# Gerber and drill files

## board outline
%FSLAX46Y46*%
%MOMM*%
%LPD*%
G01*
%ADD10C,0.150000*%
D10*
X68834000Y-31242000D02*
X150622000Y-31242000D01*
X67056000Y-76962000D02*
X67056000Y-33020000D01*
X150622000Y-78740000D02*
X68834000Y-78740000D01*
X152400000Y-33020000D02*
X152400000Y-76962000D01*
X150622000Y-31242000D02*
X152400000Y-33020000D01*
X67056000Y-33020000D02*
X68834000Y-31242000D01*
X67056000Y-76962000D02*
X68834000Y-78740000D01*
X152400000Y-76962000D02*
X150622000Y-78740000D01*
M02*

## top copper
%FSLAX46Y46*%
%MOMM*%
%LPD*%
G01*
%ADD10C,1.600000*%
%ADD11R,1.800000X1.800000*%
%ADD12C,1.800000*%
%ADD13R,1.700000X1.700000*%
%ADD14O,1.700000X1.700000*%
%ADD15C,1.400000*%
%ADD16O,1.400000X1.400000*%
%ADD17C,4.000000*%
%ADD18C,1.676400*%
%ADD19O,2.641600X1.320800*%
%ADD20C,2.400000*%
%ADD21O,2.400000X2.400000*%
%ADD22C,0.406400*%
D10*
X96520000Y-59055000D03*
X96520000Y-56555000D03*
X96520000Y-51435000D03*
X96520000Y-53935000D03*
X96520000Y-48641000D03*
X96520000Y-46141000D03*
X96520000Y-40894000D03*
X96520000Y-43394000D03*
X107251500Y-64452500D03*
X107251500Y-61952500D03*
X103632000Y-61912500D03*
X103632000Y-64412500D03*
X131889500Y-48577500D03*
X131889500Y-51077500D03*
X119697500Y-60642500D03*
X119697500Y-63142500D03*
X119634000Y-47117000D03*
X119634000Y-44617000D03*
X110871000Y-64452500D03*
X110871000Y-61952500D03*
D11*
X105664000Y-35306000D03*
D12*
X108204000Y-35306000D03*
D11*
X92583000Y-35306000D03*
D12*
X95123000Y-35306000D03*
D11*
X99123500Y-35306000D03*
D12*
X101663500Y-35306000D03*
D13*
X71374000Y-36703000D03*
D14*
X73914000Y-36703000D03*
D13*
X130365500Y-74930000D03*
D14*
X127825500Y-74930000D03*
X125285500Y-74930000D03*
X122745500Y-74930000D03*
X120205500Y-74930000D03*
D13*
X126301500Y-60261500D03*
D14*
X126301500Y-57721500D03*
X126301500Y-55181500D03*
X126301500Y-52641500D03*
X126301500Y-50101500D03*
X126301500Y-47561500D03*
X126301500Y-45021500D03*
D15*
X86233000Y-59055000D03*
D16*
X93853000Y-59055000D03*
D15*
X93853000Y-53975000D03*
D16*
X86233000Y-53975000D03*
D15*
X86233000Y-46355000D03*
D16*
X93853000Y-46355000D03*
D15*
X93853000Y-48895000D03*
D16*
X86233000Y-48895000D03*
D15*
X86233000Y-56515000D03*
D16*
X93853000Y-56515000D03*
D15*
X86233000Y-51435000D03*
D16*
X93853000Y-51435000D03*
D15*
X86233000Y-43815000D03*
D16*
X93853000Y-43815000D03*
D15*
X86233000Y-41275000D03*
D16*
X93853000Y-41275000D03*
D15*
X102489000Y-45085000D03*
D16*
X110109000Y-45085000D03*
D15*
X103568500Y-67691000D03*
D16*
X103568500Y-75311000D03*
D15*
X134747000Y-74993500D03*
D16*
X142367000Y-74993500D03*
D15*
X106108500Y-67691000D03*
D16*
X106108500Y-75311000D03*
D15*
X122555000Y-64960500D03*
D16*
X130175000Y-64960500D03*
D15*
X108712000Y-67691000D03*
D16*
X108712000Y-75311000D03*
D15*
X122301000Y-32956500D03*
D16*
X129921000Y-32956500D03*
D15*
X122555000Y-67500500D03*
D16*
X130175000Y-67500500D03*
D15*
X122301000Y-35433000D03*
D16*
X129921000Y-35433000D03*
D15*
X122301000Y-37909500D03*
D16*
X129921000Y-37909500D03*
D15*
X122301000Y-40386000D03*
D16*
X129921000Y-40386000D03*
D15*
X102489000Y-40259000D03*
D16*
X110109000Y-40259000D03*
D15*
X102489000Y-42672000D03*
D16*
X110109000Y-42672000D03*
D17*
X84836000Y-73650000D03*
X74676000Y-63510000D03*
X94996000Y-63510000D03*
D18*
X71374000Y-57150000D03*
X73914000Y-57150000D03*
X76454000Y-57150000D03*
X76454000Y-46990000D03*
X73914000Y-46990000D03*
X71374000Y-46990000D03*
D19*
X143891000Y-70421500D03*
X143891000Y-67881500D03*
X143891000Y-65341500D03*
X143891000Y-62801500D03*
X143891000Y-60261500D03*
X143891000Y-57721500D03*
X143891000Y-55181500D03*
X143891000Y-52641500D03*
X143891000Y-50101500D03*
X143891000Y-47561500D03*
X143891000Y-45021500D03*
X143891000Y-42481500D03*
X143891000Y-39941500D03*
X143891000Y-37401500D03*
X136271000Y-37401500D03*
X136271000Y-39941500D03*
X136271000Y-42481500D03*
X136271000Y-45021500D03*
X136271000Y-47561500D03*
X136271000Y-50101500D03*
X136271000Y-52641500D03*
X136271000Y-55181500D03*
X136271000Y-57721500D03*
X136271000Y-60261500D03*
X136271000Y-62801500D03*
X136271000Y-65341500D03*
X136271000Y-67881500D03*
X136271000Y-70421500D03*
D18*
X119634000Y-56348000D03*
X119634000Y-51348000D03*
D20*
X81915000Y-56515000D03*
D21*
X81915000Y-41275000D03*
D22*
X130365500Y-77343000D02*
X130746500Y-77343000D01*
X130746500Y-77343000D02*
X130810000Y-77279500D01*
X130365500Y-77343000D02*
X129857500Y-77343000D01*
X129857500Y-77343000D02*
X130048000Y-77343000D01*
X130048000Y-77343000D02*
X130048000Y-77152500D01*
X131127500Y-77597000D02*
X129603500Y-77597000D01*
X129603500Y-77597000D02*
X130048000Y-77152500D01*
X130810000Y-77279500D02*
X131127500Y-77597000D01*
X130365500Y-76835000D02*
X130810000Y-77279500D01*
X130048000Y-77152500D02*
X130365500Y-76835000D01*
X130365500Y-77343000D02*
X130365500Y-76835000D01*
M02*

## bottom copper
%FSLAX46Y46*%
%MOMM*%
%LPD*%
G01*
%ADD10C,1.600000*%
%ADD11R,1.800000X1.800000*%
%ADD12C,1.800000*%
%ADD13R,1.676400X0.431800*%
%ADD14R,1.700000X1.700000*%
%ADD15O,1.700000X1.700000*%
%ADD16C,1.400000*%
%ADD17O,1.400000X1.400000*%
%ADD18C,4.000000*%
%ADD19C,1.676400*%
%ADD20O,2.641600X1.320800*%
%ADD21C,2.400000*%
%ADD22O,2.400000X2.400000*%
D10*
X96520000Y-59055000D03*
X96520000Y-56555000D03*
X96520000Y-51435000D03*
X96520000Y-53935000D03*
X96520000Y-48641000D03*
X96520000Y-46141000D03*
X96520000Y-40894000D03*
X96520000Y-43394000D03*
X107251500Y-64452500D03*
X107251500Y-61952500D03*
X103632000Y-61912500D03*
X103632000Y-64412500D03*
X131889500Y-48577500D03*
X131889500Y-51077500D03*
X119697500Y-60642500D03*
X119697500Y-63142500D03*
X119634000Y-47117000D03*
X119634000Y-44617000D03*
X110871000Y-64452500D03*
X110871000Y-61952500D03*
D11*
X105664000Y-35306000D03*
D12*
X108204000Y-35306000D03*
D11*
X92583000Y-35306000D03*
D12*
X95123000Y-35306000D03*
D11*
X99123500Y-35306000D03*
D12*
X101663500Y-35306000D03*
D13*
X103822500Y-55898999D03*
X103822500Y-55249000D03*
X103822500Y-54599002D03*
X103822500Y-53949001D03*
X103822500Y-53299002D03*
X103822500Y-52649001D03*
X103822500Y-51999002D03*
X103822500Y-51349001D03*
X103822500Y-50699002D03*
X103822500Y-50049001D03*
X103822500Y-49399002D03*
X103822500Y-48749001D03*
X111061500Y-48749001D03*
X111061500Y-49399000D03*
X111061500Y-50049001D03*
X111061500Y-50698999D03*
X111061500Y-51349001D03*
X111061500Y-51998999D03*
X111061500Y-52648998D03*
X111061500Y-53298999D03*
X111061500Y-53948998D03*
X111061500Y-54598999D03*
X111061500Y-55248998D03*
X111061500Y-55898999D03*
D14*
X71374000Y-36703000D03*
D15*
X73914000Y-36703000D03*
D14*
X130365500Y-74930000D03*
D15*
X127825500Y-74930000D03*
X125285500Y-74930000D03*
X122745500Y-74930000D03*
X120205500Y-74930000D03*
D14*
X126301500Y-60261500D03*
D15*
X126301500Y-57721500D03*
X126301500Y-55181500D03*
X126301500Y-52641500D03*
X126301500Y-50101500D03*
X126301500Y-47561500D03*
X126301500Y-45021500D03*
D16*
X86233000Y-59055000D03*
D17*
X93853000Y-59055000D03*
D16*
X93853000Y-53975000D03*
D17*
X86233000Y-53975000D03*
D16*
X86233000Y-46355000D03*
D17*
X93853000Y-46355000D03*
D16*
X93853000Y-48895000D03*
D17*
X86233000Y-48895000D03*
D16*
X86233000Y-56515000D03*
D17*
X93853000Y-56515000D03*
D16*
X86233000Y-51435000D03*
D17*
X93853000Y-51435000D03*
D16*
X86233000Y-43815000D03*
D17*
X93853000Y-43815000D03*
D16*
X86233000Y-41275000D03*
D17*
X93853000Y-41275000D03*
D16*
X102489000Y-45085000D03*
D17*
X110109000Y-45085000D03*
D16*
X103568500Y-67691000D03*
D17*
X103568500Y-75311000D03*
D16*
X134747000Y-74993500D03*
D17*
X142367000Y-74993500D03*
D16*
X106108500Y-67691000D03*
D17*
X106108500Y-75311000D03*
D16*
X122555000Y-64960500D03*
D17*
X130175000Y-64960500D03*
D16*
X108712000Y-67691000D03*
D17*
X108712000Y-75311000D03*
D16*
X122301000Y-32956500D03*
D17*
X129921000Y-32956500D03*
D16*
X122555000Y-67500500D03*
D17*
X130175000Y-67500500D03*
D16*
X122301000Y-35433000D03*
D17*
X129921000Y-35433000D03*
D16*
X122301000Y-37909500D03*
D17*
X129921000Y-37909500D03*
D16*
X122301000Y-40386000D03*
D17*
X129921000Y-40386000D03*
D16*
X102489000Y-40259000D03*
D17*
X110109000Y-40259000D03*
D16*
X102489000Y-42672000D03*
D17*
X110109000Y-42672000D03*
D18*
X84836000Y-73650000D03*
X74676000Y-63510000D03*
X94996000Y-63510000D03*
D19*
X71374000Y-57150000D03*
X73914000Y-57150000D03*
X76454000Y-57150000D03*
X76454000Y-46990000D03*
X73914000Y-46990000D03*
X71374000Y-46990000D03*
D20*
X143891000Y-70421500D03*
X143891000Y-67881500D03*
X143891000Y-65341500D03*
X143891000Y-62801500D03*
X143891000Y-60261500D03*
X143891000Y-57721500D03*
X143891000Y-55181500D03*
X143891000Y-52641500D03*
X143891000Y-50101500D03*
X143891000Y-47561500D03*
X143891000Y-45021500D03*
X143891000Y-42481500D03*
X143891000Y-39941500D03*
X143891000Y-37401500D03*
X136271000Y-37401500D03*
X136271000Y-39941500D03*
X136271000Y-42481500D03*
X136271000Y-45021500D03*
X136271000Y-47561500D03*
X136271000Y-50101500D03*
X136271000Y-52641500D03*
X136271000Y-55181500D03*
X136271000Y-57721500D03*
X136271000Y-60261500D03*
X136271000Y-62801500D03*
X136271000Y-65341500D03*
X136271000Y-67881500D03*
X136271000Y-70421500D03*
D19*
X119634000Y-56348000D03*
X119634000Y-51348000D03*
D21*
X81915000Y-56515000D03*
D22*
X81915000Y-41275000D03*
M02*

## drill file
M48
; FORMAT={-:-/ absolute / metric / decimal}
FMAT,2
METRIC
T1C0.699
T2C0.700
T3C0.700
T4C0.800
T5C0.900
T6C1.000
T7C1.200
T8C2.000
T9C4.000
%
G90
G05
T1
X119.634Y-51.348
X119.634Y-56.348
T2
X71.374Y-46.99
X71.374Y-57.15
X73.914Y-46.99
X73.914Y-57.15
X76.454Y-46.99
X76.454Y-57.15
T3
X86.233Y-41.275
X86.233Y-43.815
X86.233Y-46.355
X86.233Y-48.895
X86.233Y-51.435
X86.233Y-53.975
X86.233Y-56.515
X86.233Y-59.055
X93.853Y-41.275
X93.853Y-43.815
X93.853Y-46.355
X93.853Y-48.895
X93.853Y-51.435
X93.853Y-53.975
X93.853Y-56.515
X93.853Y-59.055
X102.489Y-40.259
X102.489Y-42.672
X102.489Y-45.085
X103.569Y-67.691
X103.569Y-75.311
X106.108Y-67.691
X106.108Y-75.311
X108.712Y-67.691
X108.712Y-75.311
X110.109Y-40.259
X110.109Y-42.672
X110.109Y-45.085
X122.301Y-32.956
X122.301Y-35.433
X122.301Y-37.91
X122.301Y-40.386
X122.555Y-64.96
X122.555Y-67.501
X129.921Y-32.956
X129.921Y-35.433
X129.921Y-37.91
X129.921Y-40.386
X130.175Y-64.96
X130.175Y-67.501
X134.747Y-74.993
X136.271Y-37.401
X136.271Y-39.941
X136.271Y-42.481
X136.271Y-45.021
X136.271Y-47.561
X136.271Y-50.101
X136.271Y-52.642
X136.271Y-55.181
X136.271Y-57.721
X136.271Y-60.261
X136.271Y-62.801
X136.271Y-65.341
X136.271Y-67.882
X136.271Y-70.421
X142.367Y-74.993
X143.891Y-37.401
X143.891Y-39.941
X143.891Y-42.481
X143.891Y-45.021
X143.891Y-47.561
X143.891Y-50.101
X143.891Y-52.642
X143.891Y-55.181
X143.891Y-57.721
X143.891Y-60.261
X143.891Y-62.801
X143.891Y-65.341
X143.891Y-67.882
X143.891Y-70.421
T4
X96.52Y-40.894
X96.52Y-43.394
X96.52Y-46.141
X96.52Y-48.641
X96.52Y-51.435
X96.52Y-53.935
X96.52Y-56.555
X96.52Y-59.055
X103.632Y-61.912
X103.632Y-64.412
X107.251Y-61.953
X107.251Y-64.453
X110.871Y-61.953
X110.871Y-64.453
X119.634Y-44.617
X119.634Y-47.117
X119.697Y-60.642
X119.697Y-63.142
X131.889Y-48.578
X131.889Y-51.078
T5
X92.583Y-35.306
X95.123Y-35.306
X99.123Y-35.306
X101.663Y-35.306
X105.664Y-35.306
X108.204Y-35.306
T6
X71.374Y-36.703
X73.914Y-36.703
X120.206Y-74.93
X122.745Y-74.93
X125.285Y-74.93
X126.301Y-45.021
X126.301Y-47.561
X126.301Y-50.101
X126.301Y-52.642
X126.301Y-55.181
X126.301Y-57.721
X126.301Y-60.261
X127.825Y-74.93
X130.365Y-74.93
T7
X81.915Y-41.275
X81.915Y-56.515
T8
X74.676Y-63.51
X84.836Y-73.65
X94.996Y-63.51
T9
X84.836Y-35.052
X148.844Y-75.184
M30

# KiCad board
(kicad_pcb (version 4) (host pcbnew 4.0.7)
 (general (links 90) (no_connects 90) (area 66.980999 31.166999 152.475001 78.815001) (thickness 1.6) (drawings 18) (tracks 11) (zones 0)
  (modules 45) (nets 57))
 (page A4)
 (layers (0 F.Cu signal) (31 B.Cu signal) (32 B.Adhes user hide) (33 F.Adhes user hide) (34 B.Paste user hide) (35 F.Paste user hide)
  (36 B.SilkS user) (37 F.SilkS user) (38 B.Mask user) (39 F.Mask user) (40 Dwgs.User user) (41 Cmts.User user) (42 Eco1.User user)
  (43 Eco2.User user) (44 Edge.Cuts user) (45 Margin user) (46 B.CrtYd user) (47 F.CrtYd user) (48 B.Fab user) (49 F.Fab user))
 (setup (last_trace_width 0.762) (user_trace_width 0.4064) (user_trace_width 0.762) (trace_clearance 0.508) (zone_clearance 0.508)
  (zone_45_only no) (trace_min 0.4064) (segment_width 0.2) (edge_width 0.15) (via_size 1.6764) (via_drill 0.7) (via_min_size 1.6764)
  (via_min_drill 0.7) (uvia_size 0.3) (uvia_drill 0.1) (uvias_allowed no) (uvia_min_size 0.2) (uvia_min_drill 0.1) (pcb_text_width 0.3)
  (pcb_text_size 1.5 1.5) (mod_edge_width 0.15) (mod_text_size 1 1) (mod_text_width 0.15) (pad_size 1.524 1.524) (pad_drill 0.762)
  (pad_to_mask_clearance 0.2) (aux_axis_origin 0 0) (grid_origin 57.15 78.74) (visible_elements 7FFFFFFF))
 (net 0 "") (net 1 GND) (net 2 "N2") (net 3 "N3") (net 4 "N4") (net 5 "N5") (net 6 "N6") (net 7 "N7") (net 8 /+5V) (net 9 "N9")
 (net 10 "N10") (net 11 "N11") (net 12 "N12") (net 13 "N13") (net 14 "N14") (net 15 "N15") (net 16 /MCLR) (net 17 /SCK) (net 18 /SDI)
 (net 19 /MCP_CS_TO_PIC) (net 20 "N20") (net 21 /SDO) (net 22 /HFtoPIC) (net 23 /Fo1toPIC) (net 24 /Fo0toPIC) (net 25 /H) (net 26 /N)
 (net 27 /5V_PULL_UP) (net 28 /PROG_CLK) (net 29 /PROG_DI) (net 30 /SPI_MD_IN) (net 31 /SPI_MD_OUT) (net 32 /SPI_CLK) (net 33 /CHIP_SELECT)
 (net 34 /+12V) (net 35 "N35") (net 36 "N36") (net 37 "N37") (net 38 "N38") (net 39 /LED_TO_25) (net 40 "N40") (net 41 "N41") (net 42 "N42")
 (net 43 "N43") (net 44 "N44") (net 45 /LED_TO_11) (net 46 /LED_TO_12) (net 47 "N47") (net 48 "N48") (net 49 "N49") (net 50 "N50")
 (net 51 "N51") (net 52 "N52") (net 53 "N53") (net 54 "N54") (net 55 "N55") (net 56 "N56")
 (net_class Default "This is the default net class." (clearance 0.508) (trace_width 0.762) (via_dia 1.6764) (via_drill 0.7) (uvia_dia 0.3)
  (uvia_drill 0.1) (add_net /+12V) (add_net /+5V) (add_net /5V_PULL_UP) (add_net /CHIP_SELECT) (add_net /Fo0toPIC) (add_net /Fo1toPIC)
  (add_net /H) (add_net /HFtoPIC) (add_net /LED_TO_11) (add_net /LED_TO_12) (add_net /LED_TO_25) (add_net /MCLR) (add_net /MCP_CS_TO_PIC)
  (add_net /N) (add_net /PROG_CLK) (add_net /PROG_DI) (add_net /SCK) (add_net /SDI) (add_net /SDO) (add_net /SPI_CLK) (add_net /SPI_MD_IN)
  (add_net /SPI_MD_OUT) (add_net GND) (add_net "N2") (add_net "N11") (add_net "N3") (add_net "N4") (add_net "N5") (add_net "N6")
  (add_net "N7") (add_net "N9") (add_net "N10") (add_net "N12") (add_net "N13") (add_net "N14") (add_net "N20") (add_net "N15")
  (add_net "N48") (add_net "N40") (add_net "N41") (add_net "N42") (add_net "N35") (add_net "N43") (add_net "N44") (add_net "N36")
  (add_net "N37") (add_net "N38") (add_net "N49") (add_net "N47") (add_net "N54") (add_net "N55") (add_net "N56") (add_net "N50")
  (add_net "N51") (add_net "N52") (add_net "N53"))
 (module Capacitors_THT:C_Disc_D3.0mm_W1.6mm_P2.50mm (layer F.Cu) (at 96.52 59.055 90)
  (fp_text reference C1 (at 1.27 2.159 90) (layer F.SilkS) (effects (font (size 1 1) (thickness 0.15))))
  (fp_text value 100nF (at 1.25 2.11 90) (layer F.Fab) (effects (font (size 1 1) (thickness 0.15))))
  (pad 1 thru_hole circle (at 0 0 90) (size 1.6 1.6) (drill 0.8) (layers *.Cu *.Mask) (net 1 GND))
  (pad 2 thru_hole circle (at 2.5 0 90) (size 1.6 1.6) (drill 0.8) (layers *.Cu *.Mask) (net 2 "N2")))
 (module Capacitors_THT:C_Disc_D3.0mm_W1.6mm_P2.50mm (layer F.Cu) (at 96.52 51.435 270)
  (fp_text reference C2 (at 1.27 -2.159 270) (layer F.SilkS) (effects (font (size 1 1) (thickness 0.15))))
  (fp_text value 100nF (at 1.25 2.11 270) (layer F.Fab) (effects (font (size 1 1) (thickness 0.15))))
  (pad 1 thru_hole circle (at 0 0 270) (size 1.6 1.6) (drill 0.8) (layers *.Cu *.Mask) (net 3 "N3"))
  (pad 2 thru_hole circle (at 2.5 0 270) (size 1.6 1.6) (drill 0.8) (layers *.Cu *.Mask) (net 1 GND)))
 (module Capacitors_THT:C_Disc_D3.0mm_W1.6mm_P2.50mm (layer F.Cu) (at 96.52 48.641 90)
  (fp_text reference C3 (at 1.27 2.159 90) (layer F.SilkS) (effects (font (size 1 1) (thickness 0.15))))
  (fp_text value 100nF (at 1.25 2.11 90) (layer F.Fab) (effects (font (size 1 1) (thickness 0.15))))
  (pad 1 thru_hole circle (at 0 0 90) (size 1.6 1.6) (drill 0.8) (layers *.Cu *.Mask) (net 1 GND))
  (pad 2 thru_hole circle (at 2.5 0 90) (size 1.6 1.6) (drill 0.8) (layers *.Cu *.Mask) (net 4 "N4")))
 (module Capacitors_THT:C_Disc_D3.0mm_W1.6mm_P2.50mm (layer F.Cu) (at 96.52 40.894 270)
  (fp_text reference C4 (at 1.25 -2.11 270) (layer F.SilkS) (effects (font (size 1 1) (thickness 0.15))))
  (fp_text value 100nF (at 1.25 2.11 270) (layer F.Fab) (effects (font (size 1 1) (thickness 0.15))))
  (pad 1 thru_hole circle (at 0 0 270) (size 1.6 1.6) (drill 0.8) (layers *.Cu *.Mask) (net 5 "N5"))
  (pad 2 thru_hole circle (at 2.5 0 270) (size 1.6 1.6) (drill 0.8) (layers *.Cu *.Mask) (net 1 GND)))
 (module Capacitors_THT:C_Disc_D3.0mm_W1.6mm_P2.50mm (layer F.Cu) (at 107.2515 64.4525 90)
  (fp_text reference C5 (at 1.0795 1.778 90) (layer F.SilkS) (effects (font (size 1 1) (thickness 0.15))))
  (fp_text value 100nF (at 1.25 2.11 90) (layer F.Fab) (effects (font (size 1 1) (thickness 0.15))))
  (pad 1 thru_hole circle (at 0 0 90) (size 1.6 1.6) (drill 0.8) (layers *.Cu *.Mask) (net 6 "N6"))
  (pad 2 thru_hole circle (at 2.5 0 90) (size 1.6 1.6) (drill 0.8) (layers *.Cu *.Mask) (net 1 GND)))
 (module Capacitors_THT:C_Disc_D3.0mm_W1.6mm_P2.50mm (layer F.Cu) (at 103.632 61.9125 270)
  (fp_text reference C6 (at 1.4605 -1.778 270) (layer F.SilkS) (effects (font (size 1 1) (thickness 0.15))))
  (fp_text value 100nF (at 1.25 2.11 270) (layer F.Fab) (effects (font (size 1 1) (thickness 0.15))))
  (pad 1 thru_hole circle (at 0 0 270) (size 1.6 1.6) (drill 0.8) (layers *.Cu *.Mask) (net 1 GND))
  (pad 2 thru_hole circle (at 2.5 0 270) (size 1.6 1.6) (drill 0.8) (layers *.Cu *.Mask) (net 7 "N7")))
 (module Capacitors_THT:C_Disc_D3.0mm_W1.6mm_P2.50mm (layer F.Cu) (at 131.8895 48.5775 270)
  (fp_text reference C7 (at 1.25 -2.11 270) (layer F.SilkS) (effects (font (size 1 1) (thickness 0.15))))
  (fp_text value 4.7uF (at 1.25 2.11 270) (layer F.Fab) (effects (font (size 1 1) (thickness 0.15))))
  (pad 1 thru_hole circle (at 0 0 270) (size 1.6 1.6) (drill 0.8) (layers *.Cu *.Mask) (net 1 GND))
  (pad 2 thru_hole circle (at 2.5 0 270) (size 1.6 1.6) (drill 0.8) (layers *.Cu *.Mask) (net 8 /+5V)))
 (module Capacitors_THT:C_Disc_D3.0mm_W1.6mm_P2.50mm (layer F.Cu) (at 119.6975 60.6425 270)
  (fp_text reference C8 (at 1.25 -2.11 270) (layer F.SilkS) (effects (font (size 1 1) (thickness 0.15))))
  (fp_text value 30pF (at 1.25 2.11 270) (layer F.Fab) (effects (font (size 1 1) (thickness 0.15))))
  (pad 1 thru_hole circle (at 0 0 270) (size 1.6 1.6) (drill 0.8) (layers *.Cu *.Mask) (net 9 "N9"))
  (pad 2 thru_hole circle (at 2.5 0 270) (size 1.6 1.6) (drill 0.8) (layers *.Cu *.Mask) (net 1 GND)))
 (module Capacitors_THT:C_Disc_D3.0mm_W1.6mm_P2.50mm (layer F.Cu) (at 119.634 47.117 90)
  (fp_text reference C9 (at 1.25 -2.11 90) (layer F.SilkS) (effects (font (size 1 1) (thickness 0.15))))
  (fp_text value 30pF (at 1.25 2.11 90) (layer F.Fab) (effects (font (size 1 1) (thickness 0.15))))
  (pad 1 thru_hole circle (at 0 0 90) (size 1.6 1.6) (drill 0.8) (layers *.Cu *.Mask) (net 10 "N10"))
  (pad 2 thru_hole circle (at 2.5 0 90) (size 1.6 1.6) (drill 0.8) (layers *.Cu *.Mask) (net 1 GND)))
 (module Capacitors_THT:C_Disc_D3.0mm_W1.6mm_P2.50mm (layer F.Cu) (at 110.871 64.4525 90)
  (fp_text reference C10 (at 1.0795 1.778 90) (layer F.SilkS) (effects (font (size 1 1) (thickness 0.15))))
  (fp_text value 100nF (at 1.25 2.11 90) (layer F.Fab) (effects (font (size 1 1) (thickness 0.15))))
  (pad 1 thru_hole circle (at 0 0 90) (size 1.6 1.6) (drill 0.8) (layers *.Cu *.Mask) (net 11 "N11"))
  (pad 2 thru_hole circle (at 2.5 0 90) (size 1.6 1.6) (drill 0.8) (layers *.Cu *.Mask) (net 1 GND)))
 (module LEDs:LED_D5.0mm (layer F.Cu) (at 105.664 35.306)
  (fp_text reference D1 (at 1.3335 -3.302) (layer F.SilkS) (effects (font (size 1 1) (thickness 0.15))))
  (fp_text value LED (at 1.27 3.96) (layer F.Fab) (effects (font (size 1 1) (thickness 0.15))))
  (pad 1 thru_hole rect (at 0 0) (size 1.8 1.8) (drill 0.9) (layers *.Cu *.Mask) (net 1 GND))
  (pad 2 thru_hole circle (at 2.54 0) (size 1.8 1.8) (drill 0.9) (layers *.Cu *.Mask) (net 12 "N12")))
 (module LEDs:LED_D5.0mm (layer F.Cu) (at 92.583 35.306)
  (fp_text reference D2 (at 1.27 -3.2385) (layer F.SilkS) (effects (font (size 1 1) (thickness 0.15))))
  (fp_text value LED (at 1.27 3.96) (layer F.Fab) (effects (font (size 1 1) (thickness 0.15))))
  (pad 1 thru_hole rect (at 0 0) (size 1.8 1.8) (drill 0.9) (layers *.Cu *.Mask) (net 1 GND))
  (pad 2 thru_hole circle (at 2.54 0) (size 1.8 1.8) (drill 0.9) (layers *.Cu *.Mask) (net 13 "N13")))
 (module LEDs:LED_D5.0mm (layer F.Cu) (at 99.1235 35.306)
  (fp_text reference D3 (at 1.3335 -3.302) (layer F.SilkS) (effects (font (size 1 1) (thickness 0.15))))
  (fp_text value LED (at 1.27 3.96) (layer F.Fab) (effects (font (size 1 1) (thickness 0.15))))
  (pad 1 thru_hole rect (at 0 0) (size 1.8 1.8) (drill 0.9) (layers *.Cu *.Mask) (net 1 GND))
  (pad 2 thru_hole circle (at 2.54 0) (size 1.8 1.8) (drill 0.9) (layers *.Cu *.Mask) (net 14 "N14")))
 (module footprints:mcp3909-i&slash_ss (layer B.Cu) (at 107.442 52.324)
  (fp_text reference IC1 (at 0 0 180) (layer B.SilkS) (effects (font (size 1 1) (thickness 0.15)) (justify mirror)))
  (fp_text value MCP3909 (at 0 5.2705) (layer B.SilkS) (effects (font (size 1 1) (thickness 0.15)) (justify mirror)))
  (pad 1 smd rect (at -3.6195 3.574999) (size 1.6764 0.4318) (layers B.Cu B.Paste B.Mask) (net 7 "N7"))
  (pad 2 smd rect (at -3.6195 2.925) (size 1.6764 0.4318) (layers B.Cu B.Paste B.Mask) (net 7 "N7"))
  (pad 3 smd rect (at -3.6195 2.275002) (size 1.6764 0.4318) (layers B.Cu B.Paste B.Mask) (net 7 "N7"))
  (pad 4 smd rect (at -3.6195 1.625001) (size 1.6764 0.4318) (layers B.Cu B.Paste B.Mask) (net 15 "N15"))
  (pad 5 smd rect (at -3.6195 0.975002) (size 1.6764 0.4318) (layers B.Cu B.Paste B.Mask) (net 2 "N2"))
  (pad 6 smd rect (at -3.6195 0.325001) (size 1.6764 0.4318) (layers B.Cu B.Paste B.Mask) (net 3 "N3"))
  (pad 7 smd rect (at -3.6195 -0.324998) (size 1.6764 0.4318) (layers B.Cu B.Paste B.Mask) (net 4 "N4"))
  (pad 8 smd rect (at -3.6195 -0.974999) (size 1.6764 0.4318) (layers B.Cu B.Paste B.Mask) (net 5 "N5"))
  (pad 9 smd rect (at -3.6195 -1.624998) (size 1.6764 0.4318) (layers B.Cu B.Paste B.Mask) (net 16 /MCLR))
  (pad 10 smd rect (at -3.6195 -2.274999) (size 1.6764 0.4318) (layers B.Cu B.Paste B.Mask) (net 6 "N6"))
  (pad 11 smd rect (at -3.6195 -2.924998) (size 1.6764 0.4318) (layers B.Cu B.Paste B.Mask) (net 1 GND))
  (pad 12 smd rect (at -3.6195 -3.574999) (size 1.6764 0.4318) (layers B.Cu B.Paste B.Mask) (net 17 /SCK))
  (pad 13 smd rect (at 3.6195 -3.574999) (size 1.6764 0.4318) (layers B.Cu B.Paste B.Mask) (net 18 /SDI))
  (pad 14 smd rect (at 3.6195 -2.925) (size 1.6764 0.4318) (layers B.Cu B.Paste B.Mask) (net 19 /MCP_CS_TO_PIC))
  (pad 15 smd rect (at 3.6195 -2.274999) (size 1.6764 0.4318) (layers B.Cu B.Paste B.Mask) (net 1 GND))
  (pad 16 smd rect (at 3.6195 -1.625001) (size 1.6764 0.4318) (layers B.Cu B.Paste B.Mask) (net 1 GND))
  (pad 17 smd rect (at 3.6195 -0.974999) (size 1.6764 0.4318) (layers B.Cu B.Paste B.Mask) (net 10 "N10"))
  (pad 18 smd rect (at 3.6195 -0.325001) (size 1.6764 0.4318) (layers B.Cu B.Paste B.Mask) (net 9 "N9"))
  (pad 19 smd rect (at 3.6195 0.324998) (size 1.6764 0.4318) (layers B.Cu B.Paste B.Mask) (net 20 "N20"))
  (pad 20 smd rect (at 3.6195 0.974999) (size 1.6764 0.4318) (layers B.Cu B.Paste B.Mask) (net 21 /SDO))
  (pad 21 smd rect (at 3.6195 1.624998) (size 1.6764 0.4318) (layers B.Cu B.Paste B.Mask) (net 1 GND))
  (pad 22 smd rect (at 3.6195 2.274999) (size 1.6764 0.4318) (layers B.Cu B.Paste B.Mask) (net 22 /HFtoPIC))
  (pad 23 smd rect (at 3.6195 2.924998) (size 1.6764 0.4318) (layers B.Cu B.Paste B.Mask) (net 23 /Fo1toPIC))
  (pad 24 smd rect (at 3.6195 3.574999) (size 1.6764 0.4318) (layers B.Cu B.Paste B.Mask) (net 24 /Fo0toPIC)))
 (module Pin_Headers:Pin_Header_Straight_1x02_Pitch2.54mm (layer F.Cu) (at 71.374 36.703 90)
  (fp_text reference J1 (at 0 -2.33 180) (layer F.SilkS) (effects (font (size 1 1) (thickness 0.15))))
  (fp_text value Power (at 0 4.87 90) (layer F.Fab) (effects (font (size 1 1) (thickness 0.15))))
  (pad 1 thru_hole rect (at 0 0 90) (size 1.7 1.7) (drill 1) (layers *.Cu *.Mask) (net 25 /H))
  (pad 2 thru_hole oval (at 0 2.54 90) (size 1.7 1.7) (drill 1) (layers *.Cu *.Mask) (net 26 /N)))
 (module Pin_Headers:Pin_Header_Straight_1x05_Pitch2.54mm (layer F.Cu) (at 130.3655 74.93 270)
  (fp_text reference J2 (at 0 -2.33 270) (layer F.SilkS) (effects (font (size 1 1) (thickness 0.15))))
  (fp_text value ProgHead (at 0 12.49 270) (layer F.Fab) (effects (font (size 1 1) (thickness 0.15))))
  (pad 1 thru_hole rect (at 0 0 270) (size 1.7 1.7) (drill 1) (layers *.Cu *.Mask) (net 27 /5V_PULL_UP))
  (pad 2 thru_hole oval (at 0 2.54 270) (size 1.7 1.7) (drill 1) (layers *.Cu *.Mask) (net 8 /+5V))
  (pad 3 thru_hole oval (at 0 5.08 270) (size 1.7 1.7) (drill 1) (layers *.Cu *.Mask) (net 1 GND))
  (pad 4 thru_hole oval (at 0 7.62 270) (size 1.7 1.7) (drill 1) (layers *.Cu *.Mask) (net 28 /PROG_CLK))
  (pad 5 thru_hole oval (at 0 10.16 270) (size 1.7 1.7) (drill 1) (layers *.Cu *.Mask) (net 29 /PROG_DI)))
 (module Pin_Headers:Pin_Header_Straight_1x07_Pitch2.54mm (layer F.Cu) (at 126.3015 60.2615 180)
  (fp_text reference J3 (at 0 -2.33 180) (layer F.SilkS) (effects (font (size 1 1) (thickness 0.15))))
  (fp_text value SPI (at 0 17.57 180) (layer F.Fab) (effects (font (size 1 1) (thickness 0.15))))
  (pad 1 thru_hole rect (at 0 0 180) (size 1.7 1.7) (drill 1) (layers *.Cu *.Mask) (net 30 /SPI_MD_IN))
  (pad 2 thru_hole oval (at 0 2.54 180) (size 1.7 1.7) (drill 1) (layers *.Cu *.Mask) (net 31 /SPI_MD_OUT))
  (pad 3 thru_hole oval (at 0 5.08 180) (size 1.7 1.7) (drill 1) (layers *.Cu *.Mask) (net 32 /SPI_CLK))
  (pad 4 thru_hole oval (at 0 7.62 180) (size 1.7 1.7) (drill 1) (layers *.Cu *.Mask) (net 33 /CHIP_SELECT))
  (pad 5 thru_hole oval (at 0 10.16 180) (size 1.7 1.7) (drill 1) (layers *.Cu *.Mask) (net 8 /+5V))
  (pad 6 thru_hole oval (at 0 12.7 180) (size 1.7 1.7) (drill 1) (layers *.Cu *.Mask) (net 1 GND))
  (pad 7 thru_hole oval (at 0 15.24 180) (size 1.7 1.7) (drill 1) (layers *.Cu *.Mask) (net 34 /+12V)))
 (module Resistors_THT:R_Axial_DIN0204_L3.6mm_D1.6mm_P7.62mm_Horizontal (layer F.Cu) (at 86.233 59.055)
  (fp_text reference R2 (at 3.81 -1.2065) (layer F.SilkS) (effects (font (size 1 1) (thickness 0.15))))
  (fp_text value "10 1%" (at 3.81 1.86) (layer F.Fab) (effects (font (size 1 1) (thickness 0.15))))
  (pad 1 thru_hole circle (at 0 0) (size 1.4 1.4) (drill 0.7) (layers *.Cu *.Mask) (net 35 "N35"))
  (pad 2 thru_hole oval (at 7.62 0) (size 1.4 1.4) (drill 0.7) (layers *.Cu *.Mask) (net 1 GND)))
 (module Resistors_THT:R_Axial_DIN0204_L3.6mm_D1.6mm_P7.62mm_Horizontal (layer F.Cu) (at 93.853 53.975 180)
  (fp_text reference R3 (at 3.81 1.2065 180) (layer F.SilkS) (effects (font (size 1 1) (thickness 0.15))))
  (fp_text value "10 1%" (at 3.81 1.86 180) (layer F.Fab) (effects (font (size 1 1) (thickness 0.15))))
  (pad 1 thru_hole circle (at 0 0 180) (size 1.4 1.4) (drill 0.7) (layers *.Cu *.Mask) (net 1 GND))
  (pad 2 thru_hole oval (at 7.62 0 180) (size 1.4 1.4) (drill 0.7) (layers *.Cu *.Mask) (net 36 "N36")))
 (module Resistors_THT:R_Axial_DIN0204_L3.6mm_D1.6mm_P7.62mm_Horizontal (layer F.Cu) (at 86.233 46.355)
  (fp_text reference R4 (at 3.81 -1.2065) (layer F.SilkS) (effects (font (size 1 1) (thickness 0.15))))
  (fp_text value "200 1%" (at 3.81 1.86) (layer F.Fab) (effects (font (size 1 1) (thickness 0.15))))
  (pad 1 thru_hole circle (at 0 0) (size 1.4 1.4) (drill 0.7) (layers *.Cu *.Mask) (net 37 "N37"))
  (pad 2 thru_hole oval (at 7.62 0) (size 1.4 1.4) (drill 0.7) (layers *.Cu *.Mask) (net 1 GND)))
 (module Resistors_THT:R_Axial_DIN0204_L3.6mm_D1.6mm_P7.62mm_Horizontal (layer F.Cu) (at 93.853 48.895 180)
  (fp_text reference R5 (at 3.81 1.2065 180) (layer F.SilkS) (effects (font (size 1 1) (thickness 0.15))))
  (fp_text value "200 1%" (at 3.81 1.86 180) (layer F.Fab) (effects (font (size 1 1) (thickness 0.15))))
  (pad 1 thru_hole circle (at 0 0 180) (size 1.4 1.4) (drill 0.7) (layers *.Cu *.Mask) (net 1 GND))
  (pad 2 thru_hole oval (at 7.62 0 180) (size 1.4 1.4) (drill 0.7) (layers *.Cu *.Mask) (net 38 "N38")))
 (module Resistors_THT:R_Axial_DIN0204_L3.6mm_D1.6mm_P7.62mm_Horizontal (layer F.Cu) (at 86.233 56.515)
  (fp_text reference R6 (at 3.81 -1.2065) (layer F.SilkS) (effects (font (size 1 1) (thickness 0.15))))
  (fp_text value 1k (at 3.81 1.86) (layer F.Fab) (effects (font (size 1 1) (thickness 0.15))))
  (pad 1 thru_hole circle (at 0 0) (size 1.4 1.4) (drill 0.7) (layers *.Cu *.Mask) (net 35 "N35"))
  (pad 2 thru_hole oval (at 7.62 0) (size 1.4 1.4) (drill 0.7) (layers *.Cu *.Mask) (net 2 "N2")))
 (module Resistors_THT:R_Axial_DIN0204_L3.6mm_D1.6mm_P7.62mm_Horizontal (layer F.Cu) (at 86.233 51.435)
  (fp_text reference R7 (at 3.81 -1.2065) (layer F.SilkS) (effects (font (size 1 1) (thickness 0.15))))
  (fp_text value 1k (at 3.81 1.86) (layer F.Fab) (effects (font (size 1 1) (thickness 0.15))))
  (pad 1 thru_hole circle (at 0 0) (size 1.4 1.4) (drill 0.7) (layers *.Cu *.Mask) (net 36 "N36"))
  (pad 2 thru_hole oval (at 7.62 0) (size 1.4 1.4) (drill 0.7) (layers *.Cu *.Mask) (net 3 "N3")))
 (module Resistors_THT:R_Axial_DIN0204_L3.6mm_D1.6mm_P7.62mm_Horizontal (layer F.Cu) (at 86.233 43.815)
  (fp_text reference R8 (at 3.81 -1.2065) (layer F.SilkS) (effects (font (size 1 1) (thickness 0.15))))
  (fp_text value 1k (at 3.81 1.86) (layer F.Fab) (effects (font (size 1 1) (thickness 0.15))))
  (pad 1 thru_hole circle (at 0 0) (size 1.4 1.4) (drill 0.7) (layers *.Cu *.Mask) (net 37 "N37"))
  (pad 2 thru_hole oval (at 7.62 0) (size 1.4 1.4) (drill 0.7) (layers *.Cu *.Mask) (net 4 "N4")))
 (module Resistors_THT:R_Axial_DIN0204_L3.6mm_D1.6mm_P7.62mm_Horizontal (layer F.Cu) (at 86.233 41.275)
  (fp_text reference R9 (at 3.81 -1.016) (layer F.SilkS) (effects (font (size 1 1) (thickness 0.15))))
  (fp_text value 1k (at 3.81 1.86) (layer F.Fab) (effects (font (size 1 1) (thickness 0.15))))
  (pad 1 thru_hole circle (at 0 0) (size 1.4 1.4) (drill 0.7) (layers *.Cu *.Mask) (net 38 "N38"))
  (pad 2 thru_hole oval (at 7.62 0) (size 1.4 1.4) (drill 0.7) (layers *.Cu *.Mask) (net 5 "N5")))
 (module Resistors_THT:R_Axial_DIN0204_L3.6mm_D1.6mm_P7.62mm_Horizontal (layer F.Cu) (at 102.489 45.085)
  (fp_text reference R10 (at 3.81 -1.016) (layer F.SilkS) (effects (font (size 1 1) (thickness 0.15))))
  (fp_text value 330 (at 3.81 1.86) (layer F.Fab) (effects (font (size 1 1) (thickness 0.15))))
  (pad 1 thru_hole circle (at 0 0) (size 1.4 1.4) (drill 0.7) (layers *.Cu *.Mask) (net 12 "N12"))
  (pad 2 thru_hole oval (at 7.62 0) (size 1.4 1.4) (drill 0.7) (layers *.Cu *.Mask) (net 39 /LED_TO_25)))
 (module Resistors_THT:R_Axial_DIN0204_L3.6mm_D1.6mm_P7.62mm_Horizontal (layer F.Cu) (at 103.5685 67.691 270)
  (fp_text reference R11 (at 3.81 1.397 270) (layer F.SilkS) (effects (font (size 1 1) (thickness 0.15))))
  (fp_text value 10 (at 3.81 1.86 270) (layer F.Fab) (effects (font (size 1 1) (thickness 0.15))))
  (pad 1 thru_hole circle (at 0 0 270) (size 1.4 1.4) (drill 0.7) (layers *.Cu *.Mask) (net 7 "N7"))
  (pad 2 thru_hole oval (at 7.62 0 270) (size 1.4 1.4) (drill 0.7) (layers *.Cu *.Mask) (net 8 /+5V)))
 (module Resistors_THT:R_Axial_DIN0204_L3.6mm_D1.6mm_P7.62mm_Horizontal (layer F.Cu) (at 134.747 74.9935)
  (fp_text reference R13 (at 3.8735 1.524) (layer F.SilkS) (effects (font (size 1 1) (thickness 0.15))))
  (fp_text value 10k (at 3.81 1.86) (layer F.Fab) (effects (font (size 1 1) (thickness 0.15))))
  (pad 1 thru_hole circle (at 0 0) (size 1.4 1.4) (drill 0.7) (layers *.Cu *.Mask) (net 8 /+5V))
  (pad 2 thru_hole oval (at 7.62 0) (size 1.4 1.4) (drill 0.7) (layers *.Cu *.Mask) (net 27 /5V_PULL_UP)))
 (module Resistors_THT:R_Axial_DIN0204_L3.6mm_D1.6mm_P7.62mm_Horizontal (layer F.Cu) (at 106.1085 67.691 270)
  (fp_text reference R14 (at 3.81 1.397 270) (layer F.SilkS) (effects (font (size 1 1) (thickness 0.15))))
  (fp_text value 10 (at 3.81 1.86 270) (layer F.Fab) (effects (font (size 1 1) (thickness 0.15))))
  (pad 1 thru_hole circle (at 0 0 270) (size 1.4 1.4) (drill 0.7) (layers *.Cu *.Mask) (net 11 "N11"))
  (pad 2 thru_hole oval (at 7.62 0 270) (size 1.4 1.4) (drill 0.7) (layers *.Cu *.Mask) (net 8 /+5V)))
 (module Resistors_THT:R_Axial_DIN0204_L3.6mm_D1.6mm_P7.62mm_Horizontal (layer F.Cu) (at 122.555 64.9605)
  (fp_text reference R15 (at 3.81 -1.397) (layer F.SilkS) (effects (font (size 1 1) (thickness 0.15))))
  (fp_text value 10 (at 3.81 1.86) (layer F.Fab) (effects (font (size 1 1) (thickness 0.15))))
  (pad 1 thru_hole circle (at 0 0) (size 1.4 1.4) (drill 0.7) (layers *.Cu *.Mask) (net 30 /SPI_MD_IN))
  (pad 2 thru_hole oval (at 7.62 0) (size 1.4 1.4) (drill 0.7) (layers *.Cu *.Mask) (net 8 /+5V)))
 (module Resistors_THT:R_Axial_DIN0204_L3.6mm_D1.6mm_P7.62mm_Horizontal (layer F.Cu) (at 108.712 67.691 270)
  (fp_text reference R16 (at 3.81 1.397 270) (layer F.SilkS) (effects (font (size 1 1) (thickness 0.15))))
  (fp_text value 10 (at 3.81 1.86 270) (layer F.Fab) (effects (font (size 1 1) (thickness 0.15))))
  (pad 1 thru_hole circle (at 0 0 270) (size 1.4 1.4) (drill 0.7) (layers *.Cu *.Mask) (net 32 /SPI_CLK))
  (pad 2 thru_hole oval (at 7.62 0 270) (size 1.4 1.4) (drill 0.7) (layers *.Cu *.Mask) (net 8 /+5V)))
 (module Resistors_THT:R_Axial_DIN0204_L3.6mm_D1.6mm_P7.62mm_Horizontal (layer F.Cu) (at 122.301 32.9565)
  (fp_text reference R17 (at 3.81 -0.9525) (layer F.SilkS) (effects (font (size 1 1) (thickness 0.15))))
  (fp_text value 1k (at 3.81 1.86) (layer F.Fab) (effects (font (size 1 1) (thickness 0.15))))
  (pad 1 thru_hole circle (at 0 0) (size 1.4 1.4) (drill 0.7) (layers *.Cu *.Mask) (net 17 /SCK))
  (pad 2 thru_hole oval (at 7.62 0) (size 1.4 1.4) (drill 0.7) (layers *.Cu *.Mask) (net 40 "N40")))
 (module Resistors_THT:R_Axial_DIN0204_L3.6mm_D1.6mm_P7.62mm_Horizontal (layer F.Cu) (at 122.555 67.5005)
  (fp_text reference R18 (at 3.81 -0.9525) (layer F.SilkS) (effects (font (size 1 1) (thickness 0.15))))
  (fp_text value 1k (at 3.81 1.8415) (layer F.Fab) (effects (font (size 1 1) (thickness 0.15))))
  (pad 1 thru_hole circle (at 0 0) (size 1.4 1.4) (drill 0.7) (layers *.Cu *.Mask) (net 18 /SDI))
  (pad 2 thru_hole oval (at 7.62 0) (size 1.4 1.4) (drill 0.7) (layers *.Cu *.Mask) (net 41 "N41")))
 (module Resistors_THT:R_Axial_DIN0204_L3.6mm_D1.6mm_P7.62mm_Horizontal (layer F.Cu) (at 122.301 35.433)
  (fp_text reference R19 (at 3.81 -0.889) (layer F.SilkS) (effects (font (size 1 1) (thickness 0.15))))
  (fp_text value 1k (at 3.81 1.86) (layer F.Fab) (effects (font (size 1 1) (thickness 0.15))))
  (pad 1 thru_hole circle (at 0 0) (size 1.4 1.4) (drill 0.7) (layers *.Cu *.Mask) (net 21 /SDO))
  (pad 2 thru_hole oval (at 7.62 0) (size 1.4 1.4) (drill 0.7) (layers *.Cu *.Mask) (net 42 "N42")))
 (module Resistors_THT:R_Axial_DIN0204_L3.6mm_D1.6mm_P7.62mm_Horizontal (layer F.Cu) (at 122.301 37.9095)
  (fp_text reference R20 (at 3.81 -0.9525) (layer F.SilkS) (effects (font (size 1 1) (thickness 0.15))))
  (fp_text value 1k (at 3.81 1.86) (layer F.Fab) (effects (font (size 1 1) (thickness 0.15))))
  (pad 1 thru_hole circle (at 0 0) (size 1.4 1.4) (drill 0.7) (layers *.Cu *.Mask) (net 16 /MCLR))
  (pad 2 thru_hole oval (at 7.62 0) (size 1.4 1.4) (drill 0.7) (layers *.Cu *.Mask) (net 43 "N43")))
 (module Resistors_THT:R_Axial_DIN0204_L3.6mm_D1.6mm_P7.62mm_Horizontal (layer F.Cu) (at 122.301 40.386)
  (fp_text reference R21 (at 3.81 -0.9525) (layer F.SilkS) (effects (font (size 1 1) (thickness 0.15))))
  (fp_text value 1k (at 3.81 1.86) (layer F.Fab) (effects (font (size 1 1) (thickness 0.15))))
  (pad 1 thru_hole circle (at 0 0) (size 1.4 1.4) (drill 0.7) (layers *.Cu *.Mask) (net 19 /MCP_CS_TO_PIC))
  (pad 2 thru_hole oval (at 7.62 0) (size 1.4 1.4) (drill 0.7) (layers *.Cu *.Mask) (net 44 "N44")))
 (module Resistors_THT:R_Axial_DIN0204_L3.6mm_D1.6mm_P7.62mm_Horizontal (layer F.Cu) (at 102.489 40.259)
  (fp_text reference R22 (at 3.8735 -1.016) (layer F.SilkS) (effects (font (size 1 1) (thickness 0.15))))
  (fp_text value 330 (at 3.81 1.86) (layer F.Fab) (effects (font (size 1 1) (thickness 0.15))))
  (pad 1 thru_hole circle (at 0 0) (size 1.4 1.4) (drill 0.7) (layers *.Cu *.Mask) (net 13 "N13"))
  (pad 2 thru_hole oval (at 7.62 0) (size 1.4 1.4) (drill 0.7) (layers *.Cu *.Mask) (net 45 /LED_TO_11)))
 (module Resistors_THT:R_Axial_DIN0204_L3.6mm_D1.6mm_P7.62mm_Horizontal (layer F.Cu) (at 102.489 42.672)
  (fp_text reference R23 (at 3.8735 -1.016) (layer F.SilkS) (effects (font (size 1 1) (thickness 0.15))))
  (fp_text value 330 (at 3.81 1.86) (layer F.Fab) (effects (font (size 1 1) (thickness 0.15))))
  (pad 1 thru_hole circle (at 0 0) (size 1.4 1.4) (drill 0.7) (layers *.Cu *.Mask) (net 14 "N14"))
  (pad 2 thru_hole oval (at 7.62 0) (size 1.4 1.4) (drill 0.7) (layers *.Cu *.Mask) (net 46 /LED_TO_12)))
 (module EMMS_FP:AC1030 (layer F.Cu) (at 84.836 68.58 90)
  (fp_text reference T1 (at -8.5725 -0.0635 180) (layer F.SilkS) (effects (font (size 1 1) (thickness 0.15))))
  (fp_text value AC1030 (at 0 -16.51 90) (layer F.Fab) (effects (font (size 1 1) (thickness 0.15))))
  (pad 3 thru_hole circle (at -5.07 0 90) (size 4 4) (drill 2) (layers *.Cu *.Mask))
  (pad 2 thru_hole circle (at 5.07 -10.16 90) (size 4 4) (drill 2) (layers *.Cu *.Mask) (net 36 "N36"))
  (pad 1 thru_hole circle (at 5.07 10.16 90) (size 4 4) (drill 2) (layers *.Cu *.Mask) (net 35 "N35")))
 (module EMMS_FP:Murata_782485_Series (layer F.Cu) (at 73.914 52.07 270)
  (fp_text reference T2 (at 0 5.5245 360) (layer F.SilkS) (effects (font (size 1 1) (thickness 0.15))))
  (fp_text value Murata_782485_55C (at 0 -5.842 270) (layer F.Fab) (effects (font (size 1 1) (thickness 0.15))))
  (pad 4 thru_hole circle (at 5.08 2.54 270) (size 1.6764 1.6764) (drill 0.69977) (layers *.Cu *.Mask) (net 38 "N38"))
  (pad 5 thru_hole circle (at 5.08 0 270) (size 1.6764 1.6764) (drill 0.69977) (layers *.Cu *.Mask) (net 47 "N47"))
  (pad 6 thru_hole circle (at 5.08 -2.54 270) (size 1.6764 1.6764) (drill 0.69977) (layers *.Cu *.Mask) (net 37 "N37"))
  (pad 1 thru_hole circle (at -5.08 -2.54 270) (size 1.6764 1.6764) (drill 0.69977) (layers *.Cu *.Mask) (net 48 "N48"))
  (pad 2 thru_hole circle (at -5.08 0 270) (size 1.6764 1.6764) (drill 0.69977) (layers *.Cu *.Mask) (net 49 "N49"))
  (pad 3 thru_hole circle (at -5.08 2.54 270) (size 1.6764 1.6764) (drill 0.69977) (layers *.Cu *.Mask) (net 26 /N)))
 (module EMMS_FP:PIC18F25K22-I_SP (layer F.Cu) (at 143.891 70.4215 180)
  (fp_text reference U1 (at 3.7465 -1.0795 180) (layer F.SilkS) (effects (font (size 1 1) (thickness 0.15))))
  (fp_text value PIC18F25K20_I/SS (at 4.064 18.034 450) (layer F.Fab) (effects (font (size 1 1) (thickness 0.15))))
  (pad 1 thru_hole oval (at 0 0 180) (size 2.6416 1.3208) (drill 0.7) (layers *.Cu *.Mask) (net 27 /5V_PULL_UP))
  (pad 2 thru_hole oval (at 0 2.54 180) (size 2.6416 1.3208) (drill 0.7) (layers *.Cu *.Mask) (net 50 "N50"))
  (pad 3 thru_hole oval (at 0 5.08 180) (size 2.6416 1.3208) (drill 0.7) (layers *.Cu *.Mask) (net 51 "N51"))
  (pad 4 thru_hole oval (at 0 7.62 180) (size 2.6416 1.3208) (drill 0.7) (layers *.Cu *.Mask) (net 24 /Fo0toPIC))
  (pad 5 thru_hole oval (at 0 10.16 180) (size 2.6416 1.3208) (drill 0.7) (layers *.Cu *.Mask) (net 22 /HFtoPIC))
  (pad 6 thru_hole oval (at 0 12.7 180) (size 2.6416 1.3208) (drill 0.7) (layers *.Cu *.Mask) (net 23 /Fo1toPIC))
  (pad 7 thru_hole oval (at 0 15.24 180) (size 2.6416 1.3208) (drill 0.7) (layers *.Cu *.Mask) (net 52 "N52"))
  (pad 8 thru_hole oval (at 0 17.78 180) (size 2.6416 1.3208) (drill 0.7) (layers *.Cu *.Mask) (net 1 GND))
  (pad 9 thru_hole oval (at 0 20.32 180) (size 2.6416 1.3208) (drill 0.7) (layers *.Cu *.Mask) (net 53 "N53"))
  (pad 10 thru_hole oval (at 0 22.86 180) (size 2.6416 1.3208) (drill 0.7) (layers *.Cu *.Mask) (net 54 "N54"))
  (pad 11 thru_hole oval (at 0 25.4 180) (size 2.6416 1.3208) (drill 0.7) (layers *.Cu *.Mask) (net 45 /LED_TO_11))
  (pad 12 thru_hole oval (at 0 27.94 180) (size 2.6416 1.3208) (drill 0.7) (layers *.Cu *.Mask) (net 46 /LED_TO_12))
  (pad 13 thru_hole oval (at 0 30.48 180) (size 2.6416 1.3208) (drill 0.7) (layers *.Cu *.Mask) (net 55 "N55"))
  (pad 14 thru_hole oval (at 0 33.02 180) (size 2.6416 1.3208) (drill 0.7) (layers *.Cu *.Mask) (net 40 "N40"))
  (pad 15 thru_hole oval (at 7.62 33.02 180) (size 2.6416 1.3208) (drill 0.7) (layers *.Cu *.Mask) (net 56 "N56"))
  (pad 16 thru_hole oval (at 7.62 30.48 180) (size 2.6416 1.3208) (drill 0.7) (layers *.Cu *.Mask) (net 42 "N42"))
  (pad 17 thru_hole oval (at 7.62 27.94 180) (size 2.6416 1.3208) (drill 0.7) (layers *.Cu *.Mask) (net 43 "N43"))
  (pad 18 thru_hole oval (at 7.62 25.4 180) (size 2.6416 1.3208) (drill 0.7) (layers *.Cu *.Mask) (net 44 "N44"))
  (pad 19 thru_hole oval (at 7.62 22.86 180) (size 2.6416 1.3208) (drill 0.7) (layers *.Cu *.Mask) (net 1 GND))
  (pad 20 thru_hole oval (at 7.62 20.32 180) (size 2.6416 1.3208) (drill 0.7) (layers *.Cu *.Mask) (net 11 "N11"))
  (pad 21 thru_hole oval (at 7.62 17.78 180) (size 2.6416 1.3208) (drill 0.7) (layers *.Cu *.Mask) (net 33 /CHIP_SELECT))
  (pad 22 thru_hole oval (at 7.62 15.24 180) (size 2.6416 1.3208) (drill 0.7) (layers *.Cu *.Mask) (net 32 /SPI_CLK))
  (pad 23 thru_hole oval (at 7.62 12.7 180) (size 2.6416 1.3208) (drill 0.7) (layers *.Cu *.Mask) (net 31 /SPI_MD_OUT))
  (pad 24 thru_hole oval (at 7.62 10.16 180) (size 2.6416 1.3208) (drill 0.7) (layers *.Cu *.Mask) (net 30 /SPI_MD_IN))
  (pad 25 thru_hole oval (at 7.62 7.62 180) (size 2.6416 1.3208) (drill 0.7) (layers *.Cu *.Mask) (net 39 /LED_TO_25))
  (pad 26 thru_hole oval (at 7.62 5.08 180) (size 2.6416 1.3208) (drill 0.7) (layers *.Cu *.Mask) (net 41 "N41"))
  (pad 27 thru_hole oval (at 7.62 2.54 180) (size 2.6416 1.3208) (drill 0.7) (layers *.Cu *.Mask) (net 29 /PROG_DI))
  (pad 28 thru_hole oval (at 7.62 0 180) (size 2.6416 1.3208) (drill 0.7) (layers *.Cu *.Mask) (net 28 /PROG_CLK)))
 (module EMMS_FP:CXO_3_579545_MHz (layer F.Cu) (at 119.634 53.848 180)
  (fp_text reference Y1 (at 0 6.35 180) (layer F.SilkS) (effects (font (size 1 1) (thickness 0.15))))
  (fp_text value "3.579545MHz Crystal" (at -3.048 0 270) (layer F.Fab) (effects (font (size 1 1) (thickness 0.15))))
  (pad 1 thru_hole circle (at 0 -2.5 180) (size 1.6764 1.6764) (drill 0.6985) (layers *.Cu *.Mask) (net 9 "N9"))
  (pad 2 thru_hole circle (at 0 2.5 180) (size 1.6764 1.6764) (drill 0.6985) (layers *.Cu *.Mask) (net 10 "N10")))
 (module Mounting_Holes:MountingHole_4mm (layer F.Cu) (at 148.844 75.184)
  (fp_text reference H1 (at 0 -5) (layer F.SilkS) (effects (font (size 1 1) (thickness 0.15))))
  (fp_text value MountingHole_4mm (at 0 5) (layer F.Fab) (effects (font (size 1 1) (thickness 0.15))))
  (pad 1 np_thru_hole circle (at 0 0) (size 4 4) (drill 4) (layers *.Cu *.Mask)))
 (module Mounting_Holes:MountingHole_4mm (layer F.Cu) (at 84.836 35.052)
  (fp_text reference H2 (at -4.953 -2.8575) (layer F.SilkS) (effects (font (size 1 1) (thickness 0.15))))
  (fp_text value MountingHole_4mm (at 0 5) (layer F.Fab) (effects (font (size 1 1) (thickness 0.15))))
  (pad 1 np_thru_hole circle (at 0 0) (size 4 4) (drill 4) (layers *.Cu *.Mask)))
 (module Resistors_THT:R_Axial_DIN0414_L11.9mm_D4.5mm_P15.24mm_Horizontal (layer F.Cu) (at 81.915 56.515 90)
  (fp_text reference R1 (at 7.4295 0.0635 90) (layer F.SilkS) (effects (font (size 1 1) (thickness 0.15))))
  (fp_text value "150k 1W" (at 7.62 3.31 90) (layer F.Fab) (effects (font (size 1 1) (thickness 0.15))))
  (pad 1 thru_hole circle (at 0 0 90) (size 2.4 2.4) (drill 1.2) (layers *.Cu *.Mask) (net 48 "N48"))
  (pad 2 thru_hole oval (at 15.24 0 90) (size 2.4 2.4) (drill 1.2) (layers *.Cu *.Mask) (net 25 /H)))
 (gr_line (start 68.834 31.242) (end 150.622 31.242) (angle 90) (layer Edge.Cuts) (width 0.15))
 (gr_line (start 67.056 76.962) (end 67.056 33.02) (angle 90) (layer Edge.Cuts) (width 0.15))
 (gr_line (start 150.622 78.74) (end 68.834 78.74) (angle 90) (layer Edge.Cuts) (width 0.15))
 (gr_line (start 152.4 33.02) (end 152.4 76.962) (angle 90) (layer Edge.Cuts) (width 0.15))
 (gr_line (start 150.622 31.242) (end 152.4 33.02) (angle 90) (layer Edge.Cuts) (width 0.15))
 (gr_line (start 67.056 33.02) (end 68.834 31.242) (angle 90) (layer Edge.Cuts) (width 0.15))
 (gr_line (start 67.056 76.962) (end 68.834 78.74) (angle 90) (layer Edge.Cuts) (width 0.15))
 (gr_line (start 152.4 76.962) (end 150.622 78.74) (angle 90) (layer Edge.Cuts) (width 0.15))
 (segment (start 130.3655 77.343) (end 130.7465 77.343) (width 0.4064) (layer F.Cu) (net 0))
 (segment (start 130.7465 77.343) (end 130.81 77.2795) (width 0.4064) (layer F.Cu) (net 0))
 (segment (start 130.3655 77.343) (end 129.8575 77.343) (width 0.4064) (layer F.Cu) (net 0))
 (segment (start 129.8575 77.343) (end 130.048 77.343) (width 0.4064) (layer F.Cu) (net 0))
 (segment (start 130.048 77.343) (end 130.048 77.1525) (width 0.4064) (layer F.Cu) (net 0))
 (segment (start 131.1275 77.597) (end 129.6035 77.597) (width 0.4064) (layer F.Cu) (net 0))
 (segment (start 129.6035 77.597) (end 130.048 77.1525) (width 0.4064) (layer F.Cu) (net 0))
 (segment (start 130.81 77.2795) (end 131.1275 77.597) (width 0.4064) (layer F.Cu) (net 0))
 (segment (start 130.3655 76.835) (end 130.81 77.2795) (width 0.4064) (layer F.Cu) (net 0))
 (segment (start 130.048 77.1525) (end 130.3655 76.835) (width 0.4064) (layer F.Cu) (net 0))
 (segment (start 130.3655 77.343) (end 130.3655 76.835) (width 0.4064) (layer F.Cu) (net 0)))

